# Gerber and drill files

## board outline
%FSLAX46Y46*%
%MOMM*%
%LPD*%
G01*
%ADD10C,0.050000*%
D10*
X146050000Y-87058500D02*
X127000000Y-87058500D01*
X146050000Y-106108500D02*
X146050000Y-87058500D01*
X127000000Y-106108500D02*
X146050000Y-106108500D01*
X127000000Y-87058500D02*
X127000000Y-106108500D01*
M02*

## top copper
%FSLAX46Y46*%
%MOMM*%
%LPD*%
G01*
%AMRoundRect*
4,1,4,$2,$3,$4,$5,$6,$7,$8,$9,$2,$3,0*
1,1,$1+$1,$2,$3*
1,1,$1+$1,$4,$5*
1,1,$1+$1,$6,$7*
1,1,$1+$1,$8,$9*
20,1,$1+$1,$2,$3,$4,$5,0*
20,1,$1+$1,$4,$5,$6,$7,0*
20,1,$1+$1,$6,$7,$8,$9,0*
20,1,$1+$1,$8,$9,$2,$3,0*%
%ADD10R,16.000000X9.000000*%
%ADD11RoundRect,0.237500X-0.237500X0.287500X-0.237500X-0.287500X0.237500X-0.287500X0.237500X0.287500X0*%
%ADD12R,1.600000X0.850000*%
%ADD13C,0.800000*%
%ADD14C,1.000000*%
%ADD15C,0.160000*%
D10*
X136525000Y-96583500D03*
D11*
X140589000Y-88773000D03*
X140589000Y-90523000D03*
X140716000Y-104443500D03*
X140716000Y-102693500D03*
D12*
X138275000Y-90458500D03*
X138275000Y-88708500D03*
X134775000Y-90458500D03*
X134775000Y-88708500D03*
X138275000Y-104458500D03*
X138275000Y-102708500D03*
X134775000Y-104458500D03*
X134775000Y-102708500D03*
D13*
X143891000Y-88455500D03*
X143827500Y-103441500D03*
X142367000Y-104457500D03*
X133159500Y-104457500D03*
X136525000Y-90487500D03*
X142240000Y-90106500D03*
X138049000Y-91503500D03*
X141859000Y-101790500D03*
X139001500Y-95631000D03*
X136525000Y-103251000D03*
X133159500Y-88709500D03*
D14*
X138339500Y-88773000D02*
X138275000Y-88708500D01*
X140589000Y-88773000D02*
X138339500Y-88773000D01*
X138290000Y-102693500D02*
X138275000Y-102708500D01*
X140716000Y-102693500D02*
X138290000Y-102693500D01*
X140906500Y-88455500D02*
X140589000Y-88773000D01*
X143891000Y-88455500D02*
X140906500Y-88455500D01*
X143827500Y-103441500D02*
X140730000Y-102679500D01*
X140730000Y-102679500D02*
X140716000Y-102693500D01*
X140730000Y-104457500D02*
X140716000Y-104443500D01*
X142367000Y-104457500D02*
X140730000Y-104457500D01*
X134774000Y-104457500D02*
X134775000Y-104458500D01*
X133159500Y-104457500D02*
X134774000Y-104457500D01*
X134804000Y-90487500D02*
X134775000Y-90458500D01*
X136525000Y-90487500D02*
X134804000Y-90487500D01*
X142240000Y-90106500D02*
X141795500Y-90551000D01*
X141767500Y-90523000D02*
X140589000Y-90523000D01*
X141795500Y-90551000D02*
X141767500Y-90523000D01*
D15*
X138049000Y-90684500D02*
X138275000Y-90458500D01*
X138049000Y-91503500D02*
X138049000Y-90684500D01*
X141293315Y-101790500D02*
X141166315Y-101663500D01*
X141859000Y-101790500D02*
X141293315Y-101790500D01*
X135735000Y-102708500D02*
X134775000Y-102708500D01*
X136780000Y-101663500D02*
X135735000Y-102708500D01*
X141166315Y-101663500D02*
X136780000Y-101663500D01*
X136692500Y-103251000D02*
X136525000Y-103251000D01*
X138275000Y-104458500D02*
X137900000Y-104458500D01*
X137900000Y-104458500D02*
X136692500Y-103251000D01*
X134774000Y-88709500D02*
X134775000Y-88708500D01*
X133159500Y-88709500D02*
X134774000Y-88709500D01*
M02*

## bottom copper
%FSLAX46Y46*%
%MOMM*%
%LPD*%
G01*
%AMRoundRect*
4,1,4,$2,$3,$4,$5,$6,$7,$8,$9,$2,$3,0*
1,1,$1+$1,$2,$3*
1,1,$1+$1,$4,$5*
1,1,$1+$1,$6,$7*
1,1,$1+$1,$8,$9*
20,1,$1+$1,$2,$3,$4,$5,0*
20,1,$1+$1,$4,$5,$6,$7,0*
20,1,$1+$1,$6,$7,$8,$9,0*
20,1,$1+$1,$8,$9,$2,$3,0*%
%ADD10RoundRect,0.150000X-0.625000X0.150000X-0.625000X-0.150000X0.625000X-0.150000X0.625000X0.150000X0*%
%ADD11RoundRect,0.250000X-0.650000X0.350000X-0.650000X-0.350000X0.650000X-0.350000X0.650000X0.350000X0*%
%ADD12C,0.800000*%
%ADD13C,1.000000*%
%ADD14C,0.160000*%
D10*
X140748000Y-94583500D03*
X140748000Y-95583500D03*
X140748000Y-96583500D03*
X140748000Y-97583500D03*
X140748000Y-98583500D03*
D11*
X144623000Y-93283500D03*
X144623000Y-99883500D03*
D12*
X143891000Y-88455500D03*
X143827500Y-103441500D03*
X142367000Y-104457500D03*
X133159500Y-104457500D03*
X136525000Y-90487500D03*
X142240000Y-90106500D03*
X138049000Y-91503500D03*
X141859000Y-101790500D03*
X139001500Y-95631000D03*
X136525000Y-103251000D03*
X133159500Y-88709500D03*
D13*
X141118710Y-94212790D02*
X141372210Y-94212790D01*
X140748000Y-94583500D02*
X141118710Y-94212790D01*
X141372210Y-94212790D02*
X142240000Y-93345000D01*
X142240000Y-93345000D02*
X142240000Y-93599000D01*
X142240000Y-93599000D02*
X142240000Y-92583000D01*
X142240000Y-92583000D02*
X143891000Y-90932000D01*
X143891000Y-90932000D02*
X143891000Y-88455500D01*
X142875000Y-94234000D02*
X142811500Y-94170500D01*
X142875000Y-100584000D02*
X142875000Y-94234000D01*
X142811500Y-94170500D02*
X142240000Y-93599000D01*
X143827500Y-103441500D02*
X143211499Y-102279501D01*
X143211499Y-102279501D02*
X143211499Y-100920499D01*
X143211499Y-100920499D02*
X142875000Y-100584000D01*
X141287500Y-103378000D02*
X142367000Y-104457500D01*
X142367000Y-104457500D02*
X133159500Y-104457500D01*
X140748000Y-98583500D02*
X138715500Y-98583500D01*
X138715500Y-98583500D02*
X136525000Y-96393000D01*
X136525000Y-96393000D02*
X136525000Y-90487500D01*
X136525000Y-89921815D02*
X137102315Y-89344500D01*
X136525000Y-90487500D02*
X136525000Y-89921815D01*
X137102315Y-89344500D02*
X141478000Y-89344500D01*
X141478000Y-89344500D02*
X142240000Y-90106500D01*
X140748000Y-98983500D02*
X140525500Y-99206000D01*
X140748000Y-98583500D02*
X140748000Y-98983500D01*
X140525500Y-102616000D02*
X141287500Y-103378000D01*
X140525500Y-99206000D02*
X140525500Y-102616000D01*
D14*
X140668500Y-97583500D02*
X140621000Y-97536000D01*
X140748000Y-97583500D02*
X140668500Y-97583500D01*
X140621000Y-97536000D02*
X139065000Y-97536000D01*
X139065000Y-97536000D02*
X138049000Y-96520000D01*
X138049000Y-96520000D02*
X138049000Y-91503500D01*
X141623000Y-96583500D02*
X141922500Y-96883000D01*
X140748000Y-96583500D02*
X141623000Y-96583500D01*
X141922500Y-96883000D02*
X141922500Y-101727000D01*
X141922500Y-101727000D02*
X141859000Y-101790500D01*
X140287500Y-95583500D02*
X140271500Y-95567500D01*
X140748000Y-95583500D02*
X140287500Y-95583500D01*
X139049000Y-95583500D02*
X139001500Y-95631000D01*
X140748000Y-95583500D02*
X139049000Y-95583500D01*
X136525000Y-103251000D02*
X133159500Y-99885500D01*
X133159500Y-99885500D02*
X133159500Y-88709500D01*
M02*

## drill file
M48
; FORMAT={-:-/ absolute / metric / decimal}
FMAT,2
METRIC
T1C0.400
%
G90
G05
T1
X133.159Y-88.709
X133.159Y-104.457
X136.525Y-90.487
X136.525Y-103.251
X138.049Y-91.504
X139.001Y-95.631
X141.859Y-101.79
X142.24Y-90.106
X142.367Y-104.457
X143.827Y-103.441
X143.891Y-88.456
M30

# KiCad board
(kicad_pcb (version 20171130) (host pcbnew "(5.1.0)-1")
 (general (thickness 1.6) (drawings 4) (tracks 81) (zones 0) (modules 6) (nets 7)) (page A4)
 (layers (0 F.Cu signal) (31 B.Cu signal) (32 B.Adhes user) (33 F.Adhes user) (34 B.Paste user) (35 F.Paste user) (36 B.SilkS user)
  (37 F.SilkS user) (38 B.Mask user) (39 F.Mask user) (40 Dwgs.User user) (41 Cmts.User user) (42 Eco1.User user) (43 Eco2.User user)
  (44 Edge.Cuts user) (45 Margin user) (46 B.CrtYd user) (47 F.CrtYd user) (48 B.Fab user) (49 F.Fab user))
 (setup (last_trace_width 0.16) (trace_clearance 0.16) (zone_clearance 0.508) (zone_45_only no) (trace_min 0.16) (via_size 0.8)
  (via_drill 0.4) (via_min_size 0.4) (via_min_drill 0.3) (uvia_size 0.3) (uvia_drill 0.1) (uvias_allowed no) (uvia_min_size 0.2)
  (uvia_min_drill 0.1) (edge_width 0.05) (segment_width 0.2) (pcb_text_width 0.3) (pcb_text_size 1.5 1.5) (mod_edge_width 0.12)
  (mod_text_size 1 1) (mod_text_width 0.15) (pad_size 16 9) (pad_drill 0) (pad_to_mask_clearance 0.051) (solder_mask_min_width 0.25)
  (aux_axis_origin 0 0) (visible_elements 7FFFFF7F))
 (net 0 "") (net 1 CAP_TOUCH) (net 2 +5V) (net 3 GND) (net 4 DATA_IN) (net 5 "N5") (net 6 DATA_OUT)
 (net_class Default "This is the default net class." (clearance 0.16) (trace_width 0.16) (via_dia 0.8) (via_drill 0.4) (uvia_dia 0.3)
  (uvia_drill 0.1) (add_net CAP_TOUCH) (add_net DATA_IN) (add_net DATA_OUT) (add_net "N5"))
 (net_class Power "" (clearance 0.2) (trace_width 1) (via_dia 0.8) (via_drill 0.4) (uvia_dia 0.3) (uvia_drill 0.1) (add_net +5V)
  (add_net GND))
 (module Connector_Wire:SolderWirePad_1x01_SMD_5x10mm (layer F.Cu) (at 136.0805 96.647)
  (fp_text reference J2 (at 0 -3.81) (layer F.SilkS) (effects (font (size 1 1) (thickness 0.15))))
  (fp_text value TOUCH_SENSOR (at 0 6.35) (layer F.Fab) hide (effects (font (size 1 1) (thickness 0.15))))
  (pad 1 smd rect (at 0.4445 -0.0635) (size 16 9) (layers F.Cu F.Paste F.Mask) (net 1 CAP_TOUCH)))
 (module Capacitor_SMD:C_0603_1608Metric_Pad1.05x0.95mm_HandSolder (layer F.Cu) (at 140.589 89.648 270)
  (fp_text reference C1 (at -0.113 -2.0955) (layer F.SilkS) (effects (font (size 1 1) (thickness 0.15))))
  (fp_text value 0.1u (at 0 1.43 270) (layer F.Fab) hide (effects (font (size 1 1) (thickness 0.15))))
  (pad 1 smd roundrect (at -0.875 0 270) (size 1.05 0.95) (layers F.Cu F.Paste F.Mask) (roundrect_rratio 0.25) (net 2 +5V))
  (pad 2 smd roundrect (at 0.875 0 270) (size 1.05 0.95) (layers F.Cu F.Paste F.Mask) (roundrect_rratio 0.25) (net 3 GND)))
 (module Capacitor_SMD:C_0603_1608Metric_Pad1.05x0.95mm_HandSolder (layer F.Cu) (at 140.716 103.5685 270)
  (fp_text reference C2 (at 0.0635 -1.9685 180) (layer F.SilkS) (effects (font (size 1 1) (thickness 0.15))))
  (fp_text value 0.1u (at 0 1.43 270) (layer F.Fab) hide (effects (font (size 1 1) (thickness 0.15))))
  (pad 2 smd roundrect (at 0.875 0 270) (size 1.05 0.95) (layers F.Cu F.Paste F.Mask) (roundrect_rratio 0.25) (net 3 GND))
  (pad 1 smd roundrect (at -0.875 0 270) (size 1.05 0.95) (layers F.Cu F.Paste F.Mask) (roundrect_rratio 0.25) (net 2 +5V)))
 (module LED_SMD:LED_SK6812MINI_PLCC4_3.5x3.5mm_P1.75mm (layer F.Cu) (at 136.525 89.5835)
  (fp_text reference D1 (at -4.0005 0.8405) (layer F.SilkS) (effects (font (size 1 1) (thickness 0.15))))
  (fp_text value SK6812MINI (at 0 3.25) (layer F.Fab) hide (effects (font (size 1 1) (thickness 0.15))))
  (pad 3 smd rect (at 1.75 0.875) (size 1.6 0.85) (layers F.Cu F.Paste F.Mask) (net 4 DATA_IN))
  (pad 4 smd rect (at 1.75 -0.875) (size 1.6 0.85) (layers F.Cu F.Paste F.Mask) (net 2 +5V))
  (pad 2 smd rect (at -1.75 0.875) (size 1.6 0.85) (layers F.Cu F.Paste F.Mask) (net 3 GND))
  (pad 1 smd rect (at -1.75 -0.875) (size 1.6 0.85) (layers F.Cu F.Paste F.Mask) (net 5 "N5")))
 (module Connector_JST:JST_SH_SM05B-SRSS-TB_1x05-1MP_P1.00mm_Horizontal (layer B.Cu) (at 142.748 96.5835 270)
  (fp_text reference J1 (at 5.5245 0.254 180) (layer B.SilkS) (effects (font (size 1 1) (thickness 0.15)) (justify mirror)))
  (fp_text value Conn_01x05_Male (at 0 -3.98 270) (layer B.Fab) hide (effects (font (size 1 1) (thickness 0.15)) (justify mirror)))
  (pad 1 smd roundrect (at -2 2 270) (size 0.6 1.55) (layers B.Cu B.Paste B.Mask) (roundrect_rratio 0.25) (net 2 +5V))
  (pad 2 smd roundrect (at -1 2 270) (size 0.6 1.55) (layers B.Cu B.Paste B.Mask) (roundrect_rratio 0.25) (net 1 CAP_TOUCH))
  (pad 3 smd roundrect (at 0 2 270) (size 0.6 1.55) (layers B.Cu B.Paste B.Mask) (roundrect_rratio 0.25) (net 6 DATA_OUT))
  (pad 4 smd roundrect (at 1 2 270) (size 0.6 1.55) (layers B.Cu B.Paste B.Mask) (roundrect_rratio 0.25) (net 4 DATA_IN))
  (pad 5 smd roundrect (at 2 2 270) (size 0.6 1.55) (layers B.Cu B.Paste B.Mask) (roundrect_rratio 0.25) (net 3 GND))
  (pad MP smd roundrect (at -3.3 -1.875 270) (size 1.2 1.8) (layers B.Cu B.Paste B.Mask) (roundrect_rratio 0.208333))
  (pad MP smd roundrect (at 3.3 -1.875 270) (size 1.2 1.8) (layers B.Cu B.Paste B.Mask) (roundrect_rratio 0.208333)))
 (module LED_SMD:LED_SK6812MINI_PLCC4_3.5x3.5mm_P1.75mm (layer F.Cu) (at 136.525 103.5835)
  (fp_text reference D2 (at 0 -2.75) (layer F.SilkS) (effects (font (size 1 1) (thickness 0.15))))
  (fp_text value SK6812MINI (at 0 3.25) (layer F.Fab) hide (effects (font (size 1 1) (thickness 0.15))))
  (pad 3 smd rect (at 1.75 0.875) (size 1.6 0.85) (layers F.Cu F.Paste F.Mask) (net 5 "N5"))
  (pad 4 smd rect (at 1.75 -0.875) (size 1.6 0.85) (layers F.Cu F.Paste F.Mask) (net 2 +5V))
  (pad 2 smd rect (at -1.75 0.875) (size 1.6 0.85) (layers F.Cu F.Paste F.Mask) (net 3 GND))
  (pad 1 smd rect (at -1.75 -0.875) (size 1.6 0.85) (layers F.Cu F.Paste F.Mask) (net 6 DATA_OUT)))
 (gr_line (start 146.05 87.0585) (end 127 87.0585) (layer Edge.Cuts) (width 0.05))
 (gr_line (start 146.05 106.1085) (end 146.05 87.0585) (layer Edge.Cuts) (width 0.05))
 (gr_line (start 127 106.1085) (end 146.05 106.1085) (layer Edge.Cuts) (width 0.05))
 (gr_line (start 127 87.0585) (end 127 106.1085) (layer Edge.Cuts) (width 0.05))
 (segment (start 141.11871 94.21279) (end 141.37221 94.21279) (width 1) (layer B.Cu) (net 2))
 (segment (start 140.748 94.5835) (end 141.11871 94.21279) (width 1) (layer B.Cu) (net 2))
 (segment (start 141.37221 94.21279) (end 142.24 93.345) (width 1) (layer B.Cu) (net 2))
 (segment (start 138.3395 88.773) (end 138.275 88.7085) (width 1) (layer F.Cu) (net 2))
 (segment (start 140.589 88.773) (end 138.3395 88.773) (width 1) (layer F.Cu) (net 2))
 (segment (start 142.24 93.345) (end 142.24 93.599) (width 1) (layer B.Cu) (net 2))
 (segment (start 138.29 102.6935) (end 138.275 102.7085) (width 1) (layer F.Cu) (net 2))
 (segment (start 140.716 102.6935) (end 138.29 102.6935) (width 1) (layer F.Cu) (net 2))
 (segment (start 142.24 93.599) (end 142.24 92.583) (width 1) (layer B.Cu) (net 2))
 (via (at 143.891 88.4555) (size 0.8) (drill 0.4) (layers F.Cu B.Cu) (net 2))
 (segment (start 142.24 92.583) (end 143.891 90.932) (width 1) (layer B.Cu) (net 2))
 (segment (start 143.891 90.932) (end 143.891 88.4555) (width 1) (layer B.Cu) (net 2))
 (segment (start 140.9065 88.4555) (end 140.589 88.773) (width 1) (layer F.Cu) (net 2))
 (segment (start 143.891 88.4555) (end 140.9065 88.4555) (width 1) (layer F.Cu) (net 2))
 (segment (start 142.875 94.234) (end 142.8115 94.1705) (width 1) (layer B.Cu) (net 2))
 (segment (start 142.875 100.584) (end 142.875 94.234) (width 1) (layer B.Cu) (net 2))
 (segment (start 143.8275 103.4415) (end 140.73 102.6795) (width 1) (layer F.Cu) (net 2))
 (segment (start 142.8115 94.1705) (end 142.24 93.599) (width 1) (layer B.Cu) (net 2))
 (segment (start 140.73 102.6795) (end 140.716 102.6935) (width 1) (layer F.Cu) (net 2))
 (segment (start 143.8275 103.4415) (end 143.211499 102.279501) (width 1) (layer B.Cu) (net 2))
 (segment (start 143.211499 102.279501) (end 143.211499 100.920499) (width 1) (layer B.Cu) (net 2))
 (segment (start 143.211499 100.920499) (end 142.875 100.584) (width 1) (layer B.Cu) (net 2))
 (via (at 143.8275 103.4415) (size 0.8) (drill 0.4) (layers F.Cu B.Cu) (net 2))
 (via (at 142.367 104.4575) (size 0.8) (drill 0.4) (layers F.Cu B.Cu) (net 3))
 (segment (start 141.2875 103.378) (end 142.367 104.4575) (width 1) (layer B.Cu) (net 3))
 (segment (start 140.73 104.4575) (end 140.716 104.4435) (width 1) (layer F.Cu) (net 3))
 (segment (start 142.367 104.4575) (end 140.73 104.4575) (width 1) (layer F.Cu) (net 3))
 (via (at 133.1595 104.4575) (size 0.8) (drill 0.4) (layers F.Cu B.Cu) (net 3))
 (segment (start 142.367 104.4575) (end 133.1595 104.4575) (width 1) (layer B.Cu) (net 3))
 (segment (start 134.774 104.4575) (end 134.775 104.4585) (width 1) (layer F.Cu) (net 3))
 (segment (start 133.1595 104.4575) (end 134.774 104.4575) (width 1) (layer F.Cu) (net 3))
 (segment (start 140.748 98.5835) (end 138.7155 98.5835) (width 1) (layer B.Cu) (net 3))
 (via (at 136.525 90.4875) (size 0.8) (drill 0.4) (layers F.Cu B.Cu) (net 3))
 (segment (start 138.7155 98.5835) (end 136.525 96.393) (width 1) (layer B.Cu) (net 3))
 (segment (start 136.525 96.393) (end 136.525 90.4875) (width 1) (layer B.Cu) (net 3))
 (segment (start 134.804 90.4875) (end 134.775 90.4585) (width 1) (layer F.Cu) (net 3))
 (segment (start 136.525 90.4875) (end 134.804 90.4875) (width 1) (layer F.Cu) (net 3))
 (segment (start 136.525 89.921815) (end 137.102315 89.3445) (width 1) (layer B.Cu) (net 3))
 (segment (start 136.525 90.4875) (end 136.525 89.921815) (width 1) (layer B.Cu) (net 3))
 (via (at 142.24 90.1065) (size 0.8) (drill 0.4) (layers F.Cu B.Cu) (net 3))
 (segment (start 137.102315 89.3445) (end 141.478 89.3445) (width 1) (layer B.Cu) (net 3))
 (segment (start 141.478 89.3445) (end 142.24 90.1065) (width 1) (layer B.Cu) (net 3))
 (segment (start 142.24 90.1065) (end 141.7955 90.551) (width 1) (layer F.Cu) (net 3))
 (segment (start 141.7675 90.523) (end 140.589 90.523) (width 1) (layer F.Cu) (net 3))
 (segment (start 141.7955 90.551) (end 141.7675 90.523) (width 1) (layer F.Cu) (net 3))
 (segment (start 140.748 98.9835) (end 140.5255 99.206) (width 1) (layer B.Cu) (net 3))
 (segment (start 140.748 98.5835) (end 140.748 98.9835) (width 1) (layer B.Cu) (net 3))
 (segment (start 140.5255 102.616) (end 141.2875 103.378) (width 1) (layer B.Cu) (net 3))
 (segment (start 140.5255 99.206) (end 140.5255 102.616) (width 1) (layer B.Cu) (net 3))
 (segment (start 140.6685 97.5835) (end 140.621 97.536) (width 0.16) (layer B.Cu) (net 4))
 (segment (start 140.748 97.5835) (end 140.6685 97.5835) (width 0.16) (layer B.Cu) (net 4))
 (segment (start 140.621 97.536) (end 139.065 97.536) (width 0.16) (layer B.Cu) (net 4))
 (via (at 138.049 91.5035) (size 0.8) (drill 0.4) (layers F.Cu B.Cu) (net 4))
 (segment (start 139.065 97.536) (end 138.049 96.52) (width 0.16) (layer B.Cu) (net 4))
 (segment (start 138.049 96.52) (end 138.049 91.5035) (width 0.16) (layer B.Cu) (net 4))
 (segment (start 138.049 90.6845) (end 138.275 90.4585) (width 0.16) (layer F.Cu) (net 4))
 (segment (start 138.049 91.5035) (end 138.049 90.6845) (width 0.16) (layer F.Cu) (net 4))
 (segment (start 141.623 96.5835) (end 141.9225 96.883) (width 0.16) (layer B.Cu) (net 6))
 (segment (start 140.748 96.5835) (end 141.623 96.5835) (width 0.16) (layer B.Cu) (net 6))
 (via (at 141.859 101.7905) (size 0.8) (drill 0.4) (layers F.Cu B.Cu) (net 6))
 (segment (start 141.9225 96.883) (end 141.9225 101.727) (width 0.16) (layer B.Cu) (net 6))
 (segment (start 141.9225 101.727) (end 141.859 101.7905) (width 0.16) (layer B.Cu) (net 6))
 (segment (start 141.293315 101.7905) (end 141.166315 101.6635) (width 0.16) (layer F.Cu) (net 6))
 (segment (start 141.859 101.7905) (end 141.293315 101.7905) (width 0.16) (layer F.Cu) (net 6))
 (segment (start 135.735 102.7085) (end 134.775 102.7085) (width 0.16) (layer F.Cu) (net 6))
 (segment (start 136.78 101.6635) (end 135.735 102.7085) (width 0.16) (layer F.Cu) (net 6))
 (segment (start 141.166315 101.6635) (end 136.78 101.6635) (width 0.16) (layer F.Cu) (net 6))
 (segment (start 140.2875 95.5835) (end 140.2715 95.5675) (width 0.16) (layer B.Cu) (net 1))
 (segment (start 140.748 95.5835) (end 140.2875 95.5835) (width 0.16) (layer B.Cu) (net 1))
 (segment (start 139.049 95.5835) (end 139.0015 95.631) (width 0.16) (layer B.Cu) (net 1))
 (segment (start 140.748 95.5835) (end 139.049 95.5835) (width 0.16) (layer B.Cu) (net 1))
 (via (at 139.0015 95.631) (size 0.8) (drill 0.4) (layers F.Cu B.Cu) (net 1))
 (via (at 136.525 103.251) (size 0.8) (drill 0.4) (layers F.Cu B.Cu) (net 5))
 (segment (start 136.6925 103.251) (end 136.525 103.251) (width 0.16) (layer F.Cu) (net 5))
 (segment (start 138.275 104.4585) (end 137.9 104.4585) (width 0.16) (layer F.Cu) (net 5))
 (segment (start 137.9 104.4585) (end 136.6925 103.251) (width 0.16) (layer F.Cu) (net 5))
 (via (at 133.1595 88.7095) (size 0.8) (drill 0.4) (layers F.Cu B.Cu) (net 5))
 (segment (start 136.525 103.251) (end 133.1595 99.8855) (width 0.16) (layer B.Cu) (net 5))
 (segment (start 133.1595 99.8855) (end 133.1595 88.7095) (width 0.16) (layer B.Cu) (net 5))
 (segment (start 134.774 88.7095) (end 134.775 88.7085) (width 0.16) (layer F.Cu) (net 5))
 (segment (start 133.1595 88.7095) (end 134.774 88.7095) (width 0.16) (layer F.Cu) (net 5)))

